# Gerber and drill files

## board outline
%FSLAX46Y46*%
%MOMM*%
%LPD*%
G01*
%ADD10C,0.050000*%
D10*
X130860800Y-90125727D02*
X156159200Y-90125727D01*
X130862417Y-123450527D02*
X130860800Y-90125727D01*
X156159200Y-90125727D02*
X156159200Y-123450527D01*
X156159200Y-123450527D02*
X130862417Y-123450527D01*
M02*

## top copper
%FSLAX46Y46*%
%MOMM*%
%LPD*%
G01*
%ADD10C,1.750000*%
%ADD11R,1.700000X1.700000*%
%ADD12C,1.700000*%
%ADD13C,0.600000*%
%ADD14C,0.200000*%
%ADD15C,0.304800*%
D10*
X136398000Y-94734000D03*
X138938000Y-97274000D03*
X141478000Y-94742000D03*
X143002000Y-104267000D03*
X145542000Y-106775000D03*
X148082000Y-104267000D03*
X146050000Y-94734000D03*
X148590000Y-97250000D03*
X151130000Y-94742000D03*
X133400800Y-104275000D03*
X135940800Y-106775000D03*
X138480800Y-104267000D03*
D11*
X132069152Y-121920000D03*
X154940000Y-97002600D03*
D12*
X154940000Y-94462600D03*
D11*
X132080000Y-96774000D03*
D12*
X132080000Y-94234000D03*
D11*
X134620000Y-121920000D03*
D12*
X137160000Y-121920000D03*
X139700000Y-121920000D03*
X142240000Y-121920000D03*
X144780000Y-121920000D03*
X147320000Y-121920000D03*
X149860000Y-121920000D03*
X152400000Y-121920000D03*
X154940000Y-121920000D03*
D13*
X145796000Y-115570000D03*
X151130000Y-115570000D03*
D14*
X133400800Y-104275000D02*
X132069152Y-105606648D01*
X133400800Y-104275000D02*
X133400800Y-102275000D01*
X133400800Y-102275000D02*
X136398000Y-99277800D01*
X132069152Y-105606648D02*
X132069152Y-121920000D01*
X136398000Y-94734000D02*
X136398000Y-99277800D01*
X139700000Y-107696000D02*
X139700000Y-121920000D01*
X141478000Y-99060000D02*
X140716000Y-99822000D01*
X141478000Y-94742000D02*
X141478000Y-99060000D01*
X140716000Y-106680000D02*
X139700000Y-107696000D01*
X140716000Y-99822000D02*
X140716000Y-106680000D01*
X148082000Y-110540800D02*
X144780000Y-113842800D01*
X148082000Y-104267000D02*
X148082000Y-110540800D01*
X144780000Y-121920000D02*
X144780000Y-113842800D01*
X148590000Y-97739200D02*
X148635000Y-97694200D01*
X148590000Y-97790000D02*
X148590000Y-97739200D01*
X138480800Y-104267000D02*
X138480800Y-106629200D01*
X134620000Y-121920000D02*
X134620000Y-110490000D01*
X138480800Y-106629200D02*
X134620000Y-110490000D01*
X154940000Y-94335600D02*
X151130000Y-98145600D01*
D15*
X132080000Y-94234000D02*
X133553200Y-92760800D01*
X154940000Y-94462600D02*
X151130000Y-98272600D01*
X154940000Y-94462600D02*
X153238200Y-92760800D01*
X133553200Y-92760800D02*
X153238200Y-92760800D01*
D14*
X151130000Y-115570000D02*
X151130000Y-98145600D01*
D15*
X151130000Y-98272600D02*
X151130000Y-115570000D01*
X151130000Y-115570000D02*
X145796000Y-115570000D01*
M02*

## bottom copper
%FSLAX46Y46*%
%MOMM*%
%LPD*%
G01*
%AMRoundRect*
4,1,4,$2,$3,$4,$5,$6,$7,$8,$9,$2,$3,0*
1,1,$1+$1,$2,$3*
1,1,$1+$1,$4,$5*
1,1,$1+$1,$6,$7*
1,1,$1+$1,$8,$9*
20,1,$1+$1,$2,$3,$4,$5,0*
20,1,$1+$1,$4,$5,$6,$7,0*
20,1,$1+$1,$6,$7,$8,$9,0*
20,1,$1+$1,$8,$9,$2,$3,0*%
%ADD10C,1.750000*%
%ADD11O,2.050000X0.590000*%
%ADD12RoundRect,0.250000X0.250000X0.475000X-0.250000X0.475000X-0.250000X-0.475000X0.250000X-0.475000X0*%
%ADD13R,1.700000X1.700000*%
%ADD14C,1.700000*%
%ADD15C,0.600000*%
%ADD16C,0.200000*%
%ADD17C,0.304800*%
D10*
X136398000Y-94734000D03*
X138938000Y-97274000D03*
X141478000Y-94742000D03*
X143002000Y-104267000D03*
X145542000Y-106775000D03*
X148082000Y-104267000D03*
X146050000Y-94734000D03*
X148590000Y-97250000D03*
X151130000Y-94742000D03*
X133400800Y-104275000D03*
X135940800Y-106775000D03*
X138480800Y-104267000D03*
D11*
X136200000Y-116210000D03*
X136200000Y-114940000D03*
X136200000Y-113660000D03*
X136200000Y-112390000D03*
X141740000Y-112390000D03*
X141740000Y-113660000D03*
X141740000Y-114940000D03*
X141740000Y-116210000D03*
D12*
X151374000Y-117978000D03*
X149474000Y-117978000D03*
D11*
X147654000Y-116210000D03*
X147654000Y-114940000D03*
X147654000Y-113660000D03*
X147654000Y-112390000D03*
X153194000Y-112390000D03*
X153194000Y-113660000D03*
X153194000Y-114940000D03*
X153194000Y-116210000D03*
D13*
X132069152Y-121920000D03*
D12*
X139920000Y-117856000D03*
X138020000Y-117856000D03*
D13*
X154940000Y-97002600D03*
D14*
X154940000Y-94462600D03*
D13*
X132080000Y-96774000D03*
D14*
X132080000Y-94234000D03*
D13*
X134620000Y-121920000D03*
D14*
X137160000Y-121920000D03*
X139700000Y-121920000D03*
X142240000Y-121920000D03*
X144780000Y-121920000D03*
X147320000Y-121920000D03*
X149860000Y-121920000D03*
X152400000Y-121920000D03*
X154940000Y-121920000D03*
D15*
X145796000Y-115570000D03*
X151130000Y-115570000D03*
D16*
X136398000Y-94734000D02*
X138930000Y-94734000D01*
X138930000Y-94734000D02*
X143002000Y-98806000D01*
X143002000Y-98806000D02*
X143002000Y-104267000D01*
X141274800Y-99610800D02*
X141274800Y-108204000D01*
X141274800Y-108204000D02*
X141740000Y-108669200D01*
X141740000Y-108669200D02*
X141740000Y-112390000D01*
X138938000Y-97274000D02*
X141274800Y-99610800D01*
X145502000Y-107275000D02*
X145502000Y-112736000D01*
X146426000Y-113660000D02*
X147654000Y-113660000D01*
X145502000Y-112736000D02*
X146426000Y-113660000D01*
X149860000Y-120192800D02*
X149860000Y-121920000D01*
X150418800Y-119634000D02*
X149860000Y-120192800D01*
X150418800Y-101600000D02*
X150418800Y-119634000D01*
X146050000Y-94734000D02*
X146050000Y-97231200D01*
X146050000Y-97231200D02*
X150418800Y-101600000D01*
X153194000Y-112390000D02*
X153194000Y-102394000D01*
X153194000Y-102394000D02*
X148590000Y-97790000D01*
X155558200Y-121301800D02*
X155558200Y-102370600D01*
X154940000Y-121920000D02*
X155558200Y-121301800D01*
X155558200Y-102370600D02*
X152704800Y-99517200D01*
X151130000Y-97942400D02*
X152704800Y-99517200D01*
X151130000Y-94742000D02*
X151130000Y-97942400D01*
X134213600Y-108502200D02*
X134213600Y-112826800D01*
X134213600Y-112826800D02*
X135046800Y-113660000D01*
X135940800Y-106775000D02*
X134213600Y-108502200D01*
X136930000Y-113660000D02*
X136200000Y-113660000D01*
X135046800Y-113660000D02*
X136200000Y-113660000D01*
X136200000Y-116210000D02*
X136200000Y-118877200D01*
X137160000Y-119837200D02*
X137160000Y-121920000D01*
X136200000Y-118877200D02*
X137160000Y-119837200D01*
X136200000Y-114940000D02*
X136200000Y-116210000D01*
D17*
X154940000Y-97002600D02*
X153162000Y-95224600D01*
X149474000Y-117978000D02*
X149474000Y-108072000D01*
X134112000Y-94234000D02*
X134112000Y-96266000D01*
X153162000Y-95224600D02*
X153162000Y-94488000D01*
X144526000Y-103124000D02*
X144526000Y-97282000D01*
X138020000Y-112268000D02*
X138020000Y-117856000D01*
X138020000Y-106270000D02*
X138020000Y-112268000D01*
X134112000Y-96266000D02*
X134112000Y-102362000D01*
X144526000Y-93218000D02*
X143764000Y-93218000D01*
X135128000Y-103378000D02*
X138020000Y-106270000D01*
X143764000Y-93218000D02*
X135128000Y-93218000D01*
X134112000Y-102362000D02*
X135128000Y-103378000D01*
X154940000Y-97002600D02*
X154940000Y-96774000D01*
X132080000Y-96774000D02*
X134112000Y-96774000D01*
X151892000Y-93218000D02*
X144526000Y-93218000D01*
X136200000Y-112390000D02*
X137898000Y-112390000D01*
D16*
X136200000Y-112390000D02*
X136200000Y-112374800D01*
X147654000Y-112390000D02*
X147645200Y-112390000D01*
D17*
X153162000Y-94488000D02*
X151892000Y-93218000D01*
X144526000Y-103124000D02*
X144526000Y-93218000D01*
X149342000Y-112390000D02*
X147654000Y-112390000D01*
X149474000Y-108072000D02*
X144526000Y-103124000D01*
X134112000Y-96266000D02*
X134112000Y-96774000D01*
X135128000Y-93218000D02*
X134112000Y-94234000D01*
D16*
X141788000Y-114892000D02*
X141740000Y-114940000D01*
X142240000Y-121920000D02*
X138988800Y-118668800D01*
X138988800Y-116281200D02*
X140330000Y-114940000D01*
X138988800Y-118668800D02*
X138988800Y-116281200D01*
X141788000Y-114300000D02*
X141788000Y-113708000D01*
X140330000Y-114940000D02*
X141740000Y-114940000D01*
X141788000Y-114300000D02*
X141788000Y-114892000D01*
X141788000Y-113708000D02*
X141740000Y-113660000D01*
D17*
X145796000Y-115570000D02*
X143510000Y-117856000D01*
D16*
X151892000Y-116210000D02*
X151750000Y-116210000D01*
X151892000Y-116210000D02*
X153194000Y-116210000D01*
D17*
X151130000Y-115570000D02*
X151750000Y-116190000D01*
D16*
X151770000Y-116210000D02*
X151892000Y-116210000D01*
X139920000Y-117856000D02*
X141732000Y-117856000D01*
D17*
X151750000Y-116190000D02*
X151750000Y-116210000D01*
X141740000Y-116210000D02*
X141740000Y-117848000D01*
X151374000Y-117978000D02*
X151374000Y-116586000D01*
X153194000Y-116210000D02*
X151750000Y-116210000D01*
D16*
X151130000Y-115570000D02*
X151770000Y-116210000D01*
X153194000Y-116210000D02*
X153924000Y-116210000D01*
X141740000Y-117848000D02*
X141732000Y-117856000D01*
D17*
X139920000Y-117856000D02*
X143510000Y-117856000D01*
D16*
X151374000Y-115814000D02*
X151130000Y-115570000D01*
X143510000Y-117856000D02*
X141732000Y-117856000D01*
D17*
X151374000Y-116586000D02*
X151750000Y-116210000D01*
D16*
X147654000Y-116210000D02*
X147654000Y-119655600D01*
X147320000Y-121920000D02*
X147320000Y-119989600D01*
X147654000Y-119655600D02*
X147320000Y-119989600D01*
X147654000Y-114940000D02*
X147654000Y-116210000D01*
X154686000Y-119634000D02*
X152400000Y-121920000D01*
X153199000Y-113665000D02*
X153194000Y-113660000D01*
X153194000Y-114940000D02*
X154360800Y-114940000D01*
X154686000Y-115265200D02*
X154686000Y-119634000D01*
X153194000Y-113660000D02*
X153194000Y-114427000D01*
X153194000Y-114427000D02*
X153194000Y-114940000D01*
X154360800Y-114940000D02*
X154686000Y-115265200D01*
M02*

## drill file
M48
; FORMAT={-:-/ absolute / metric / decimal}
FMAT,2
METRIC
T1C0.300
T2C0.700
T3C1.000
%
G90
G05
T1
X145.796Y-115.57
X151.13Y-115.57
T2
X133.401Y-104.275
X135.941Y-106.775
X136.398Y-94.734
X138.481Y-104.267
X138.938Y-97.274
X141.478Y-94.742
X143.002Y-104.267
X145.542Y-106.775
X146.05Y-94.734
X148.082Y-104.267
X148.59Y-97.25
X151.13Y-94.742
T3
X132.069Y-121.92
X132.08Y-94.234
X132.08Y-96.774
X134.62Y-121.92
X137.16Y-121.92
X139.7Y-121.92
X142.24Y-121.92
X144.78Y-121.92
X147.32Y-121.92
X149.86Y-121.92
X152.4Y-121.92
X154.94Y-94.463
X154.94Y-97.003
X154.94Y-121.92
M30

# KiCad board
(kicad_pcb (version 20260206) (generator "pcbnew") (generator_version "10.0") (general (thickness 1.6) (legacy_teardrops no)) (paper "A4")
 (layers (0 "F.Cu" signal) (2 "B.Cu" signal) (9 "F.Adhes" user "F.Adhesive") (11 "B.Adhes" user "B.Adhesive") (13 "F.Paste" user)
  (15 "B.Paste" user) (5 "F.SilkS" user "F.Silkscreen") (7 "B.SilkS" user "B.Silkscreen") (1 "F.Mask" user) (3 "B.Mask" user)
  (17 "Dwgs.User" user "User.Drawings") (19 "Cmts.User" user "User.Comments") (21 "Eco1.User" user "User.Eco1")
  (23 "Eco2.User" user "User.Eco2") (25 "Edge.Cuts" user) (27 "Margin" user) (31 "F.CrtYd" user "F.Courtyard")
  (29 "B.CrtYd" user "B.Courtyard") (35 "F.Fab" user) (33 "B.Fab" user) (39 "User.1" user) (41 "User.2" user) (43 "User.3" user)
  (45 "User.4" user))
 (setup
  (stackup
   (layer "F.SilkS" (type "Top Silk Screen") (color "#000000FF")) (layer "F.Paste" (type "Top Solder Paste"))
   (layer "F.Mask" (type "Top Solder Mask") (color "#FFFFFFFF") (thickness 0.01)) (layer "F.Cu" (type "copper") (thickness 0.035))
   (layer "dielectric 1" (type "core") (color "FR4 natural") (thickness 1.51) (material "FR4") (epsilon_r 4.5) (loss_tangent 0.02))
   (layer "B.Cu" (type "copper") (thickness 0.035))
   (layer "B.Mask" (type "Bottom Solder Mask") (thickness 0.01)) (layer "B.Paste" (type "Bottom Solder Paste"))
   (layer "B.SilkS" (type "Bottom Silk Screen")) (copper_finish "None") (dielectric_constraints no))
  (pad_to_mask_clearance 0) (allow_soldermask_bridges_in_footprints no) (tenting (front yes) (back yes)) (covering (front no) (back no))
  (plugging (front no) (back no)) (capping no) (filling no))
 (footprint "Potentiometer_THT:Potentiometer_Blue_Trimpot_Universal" (layer "F.Cu") (at 141.478 95.242 90)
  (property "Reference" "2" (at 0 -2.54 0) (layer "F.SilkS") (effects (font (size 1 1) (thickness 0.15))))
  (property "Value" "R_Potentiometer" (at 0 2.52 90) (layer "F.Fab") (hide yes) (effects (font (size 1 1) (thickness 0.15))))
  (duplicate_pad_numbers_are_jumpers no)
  (pad "1" thru_hole circle (at 0.508 -5.08 90) (size 1.75 1.75) (drill 0.7) (layers "*.Cu" "*.Mask") (remove_unused_layers no)
   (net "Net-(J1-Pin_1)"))
  (pad "2" thru_hole circle (at -2.032 -2.54 90) (size 1.75 1.75) (drill 0.7) (layers "*.Cu" "*.Mask") (remove_unused_layers no)
   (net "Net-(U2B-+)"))
  (pad "3" thru_hole circle (at 0.5 0 90) (size 1.75 1.75) (drill 0.7) (layers "*.Cu" "*.Mask") (remove_unused_layers no)
   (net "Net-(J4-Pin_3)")))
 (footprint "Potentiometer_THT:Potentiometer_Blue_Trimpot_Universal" (layer "F.Cu") (at 148.082 104.775 90)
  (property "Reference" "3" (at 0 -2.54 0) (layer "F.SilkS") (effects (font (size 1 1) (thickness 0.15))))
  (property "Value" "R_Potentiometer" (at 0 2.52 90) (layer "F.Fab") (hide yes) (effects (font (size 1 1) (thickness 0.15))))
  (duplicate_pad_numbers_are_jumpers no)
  (pad "1" thru_hole circle (at 0.508 -5.08 90) (size 1.75 1.75) (drill 0.7) (layers "*.Cu" "*.Mask") (remove_unused_layers no)
   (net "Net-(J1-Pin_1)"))
  (pad "2" thru_hole circle (at -2 -2.54 90) (size 1.75 1.75) (drill 0.7) (layers "*.Cu" "*.Mask") (remove_unused_layers no)
   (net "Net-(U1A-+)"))
  (pad "3" thru_hole circle (at 0.508 0 90) (size 1.75 1.75) (drill 0.7) (layers "*.Cu" "*.Mask") (remove_unused_layers no)
   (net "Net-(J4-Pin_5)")))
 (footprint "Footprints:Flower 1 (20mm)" (layer "F.Cu") (at 154.2796 110.744)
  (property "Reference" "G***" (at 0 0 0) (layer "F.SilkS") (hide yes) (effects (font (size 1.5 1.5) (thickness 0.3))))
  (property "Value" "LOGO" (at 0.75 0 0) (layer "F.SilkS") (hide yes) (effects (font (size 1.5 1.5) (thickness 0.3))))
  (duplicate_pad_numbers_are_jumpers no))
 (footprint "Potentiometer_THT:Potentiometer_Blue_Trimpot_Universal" (layer "F.Cu") (at 151.13 95.25 90)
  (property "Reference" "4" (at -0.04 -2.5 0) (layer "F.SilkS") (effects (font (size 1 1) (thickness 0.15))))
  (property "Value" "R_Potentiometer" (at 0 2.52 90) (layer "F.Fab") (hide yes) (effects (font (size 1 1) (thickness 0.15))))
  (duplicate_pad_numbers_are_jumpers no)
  (pad "1" thru_hole circle (at 0.516 -5.08 90) (size 1.75 1.75) (drill 0.7) (layers "*.Cu" "*.Mask") (remove_unused_layers no)
   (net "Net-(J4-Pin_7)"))
  (pad "2" thru_hole circle (at -2 -2.54 90) (size 1.75 1.75) (drill 0.7) (layers "*.Cu" "*.Mask") (remove_unused_layers no)
   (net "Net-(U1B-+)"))
  (pad "3" thru_hole circle (at 0.508 0 90) (size 1.75 1.75) (drill 0.7) (layers "*.Cu" "*.Mask") (remove_unused_layers no)
   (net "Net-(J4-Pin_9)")))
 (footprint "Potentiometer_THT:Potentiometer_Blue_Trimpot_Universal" (layer "F.Cu") (at 138.4808 104.775 90)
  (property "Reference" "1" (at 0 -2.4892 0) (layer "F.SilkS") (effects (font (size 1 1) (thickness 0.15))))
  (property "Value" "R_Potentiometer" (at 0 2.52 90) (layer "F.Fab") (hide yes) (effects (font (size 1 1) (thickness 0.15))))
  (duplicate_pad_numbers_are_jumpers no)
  (pad "1" thru_hole circle (at 0.5 -5.08 90) (size 1.75 1.75) (drill 0.7) (layers "*.Cu" "*.Mask") (remove_unused_layers no)
   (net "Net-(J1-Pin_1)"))
  (pad "2" thru_hole circle (at -2 -2.54 90) (size 1.75 1.75) (drill 0.7) (layers "*.Cu" "*.Mask") (remove_unused_layers no)
   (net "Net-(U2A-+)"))
  (pad "3" thru_hole circle (at 0.508 0 90) (size 1.75 1.75) (drill 0.7) (layers "*.Cu" "*.Mask") (remove_unused_layers no)
   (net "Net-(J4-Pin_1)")))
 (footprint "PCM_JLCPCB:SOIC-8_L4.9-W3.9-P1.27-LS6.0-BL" (layer "B.Cu") (at 138.97 114.3 90)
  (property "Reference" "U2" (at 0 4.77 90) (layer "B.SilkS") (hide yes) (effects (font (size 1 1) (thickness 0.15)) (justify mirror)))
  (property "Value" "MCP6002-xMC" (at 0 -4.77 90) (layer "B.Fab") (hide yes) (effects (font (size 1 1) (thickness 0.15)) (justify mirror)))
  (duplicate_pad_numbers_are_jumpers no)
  (pad "1" smd oval (at -1.91 -2.77 90) (size 0.59 2.05) (layers "B.Cu" "B.Mask" "B.Paste") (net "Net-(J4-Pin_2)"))
  (pad "2" smd oval (at -0.64 -2.77 90) (size 0.59 2.05) (layers "B.Cu" "B.Mask" "B.Paste") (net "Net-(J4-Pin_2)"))
  (pad "3" smd oval (at 0.64 -2.77 90) (size 0.59 2.05) (layers "B.Cu" "B.Mask" "B.Paste") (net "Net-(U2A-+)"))
  (pad "4" smd oval (at 1.91 -2.77 90) (size 0.59 2.05) (layers "B.Cu" "B.Mask" "B.Paste") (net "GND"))
  (pad "5" smd oval (at 1.91 2.77 90) (size 0.59 2.05) (layers "B.Cu" "B.Mask" "B.Paste") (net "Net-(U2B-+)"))
  (pad "6" smd oval (at 0.64 2.77 90) (size 0.59 2.05) (layers "B.Cu" "B.Mask" "B.Paste") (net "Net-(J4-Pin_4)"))
  (pad "7" smd oval (at -0.64 2.77 90) (size 0.59 2.05) (layers "B.Cu" "B.Mask" "B.Paste") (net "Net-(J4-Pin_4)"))
  (pad "8" smd oval (at -1.91 2.77 90) (size 0.59 2.05) (layers "B.Cu" "B.Mask" "B.Paste") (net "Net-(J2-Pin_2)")))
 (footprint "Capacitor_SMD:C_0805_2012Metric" (layer "B.Cu") (at 150.424 117.978 180)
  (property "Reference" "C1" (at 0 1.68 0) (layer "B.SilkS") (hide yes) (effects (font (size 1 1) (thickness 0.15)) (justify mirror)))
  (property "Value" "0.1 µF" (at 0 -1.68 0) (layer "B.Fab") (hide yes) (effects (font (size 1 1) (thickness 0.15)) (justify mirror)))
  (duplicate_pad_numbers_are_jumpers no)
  (pad "1" smd roundrect (at -0.95 0 180) (size 1 1.45) (layers "B.Cu" "B.Mask" "B.Paste") (roundrect_rratio 0.25) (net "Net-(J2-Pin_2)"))
  (pad "2" smd roundrect (at 0.95 0 180) (size 1 1.45) (layers "B.Cu" "B.Mask" "B.Paste") (roundrect_rratio 0.25) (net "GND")))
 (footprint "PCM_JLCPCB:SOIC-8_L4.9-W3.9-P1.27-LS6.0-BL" (layer "B.Cu") (at 150.424 114.3 90)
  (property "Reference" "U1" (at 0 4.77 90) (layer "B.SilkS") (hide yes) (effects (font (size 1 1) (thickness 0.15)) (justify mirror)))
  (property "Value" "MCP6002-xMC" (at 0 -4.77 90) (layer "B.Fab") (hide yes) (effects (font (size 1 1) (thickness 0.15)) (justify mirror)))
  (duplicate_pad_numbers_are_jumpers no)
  (pad "1" smd oval (at -1.91 -2.77 90) (size 0.59 2.05) (layers "B.Cu" "B.Mask" "B.Paste") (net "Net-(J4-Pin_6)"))
  (pad "2" smd oval (at -0.64 -2.77 90) (size 0.59 2.05) (layers "B.Cu" "B.Mask" "B.Paste") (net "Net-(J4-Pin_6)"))
  (pad "3" smd oval (at 0.64 -2.77 90) (size 0.59 2.05) (layers "B.Cu" "B.Mask" "B.Paste") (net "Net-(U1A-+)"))
  (pad "4" smd oval (at 1.91 -2.77 90) (size 0.59 2.05) (layers "B.Cu" "B.Mask" "B.Paste") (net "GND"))
  (pad "5" smd oval (at 1.91 2.77 90) (size 0.59 2.05) (layers "B.Cu" "B.Mask" "B.Paste") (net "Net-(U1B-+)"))
  (pad "6" smd oval (at 0.64 2.77 90) (size 0.59 2.05) (layers "B.Cu" "B.Mask" "B.Paste") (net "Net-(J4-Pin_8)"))
  (pad "7" smd oval (at -0.64 2.77 90) (size 0.59 2.05) (layers "B.Cu" "B.Mask" "B.Paste") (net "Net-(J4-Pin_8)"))
  (pad "8" smd oval (at -1.91 2.77 90) (size 0.59 2.05) (layers "B.Cu" "B.Mask" "B.Paste") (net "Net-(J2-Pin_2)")))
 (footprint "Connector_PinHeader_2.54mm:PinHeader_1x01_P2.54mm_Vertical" (layer "B.Cu") (at 132.069152 121.92 -90)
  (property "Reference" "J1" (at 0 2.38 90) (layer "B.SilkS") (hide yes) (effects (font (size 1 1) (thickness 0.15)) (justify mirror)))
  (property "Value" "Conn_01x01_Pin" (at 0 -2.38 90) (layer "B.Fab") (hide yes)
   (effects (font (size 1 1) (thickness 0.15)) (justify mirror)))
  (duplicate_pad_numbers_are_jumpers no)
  (pad "1" thru_hole rect (at 0 0 270) (size 1.7 1.7) (drill 1) (layers "*.Cu" "*.Mask") (remove_unused_layers no) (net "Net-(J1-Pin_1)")))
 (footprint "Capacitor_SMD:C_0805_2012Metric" (layer "B.Cu") (at 138.97 117.856 180)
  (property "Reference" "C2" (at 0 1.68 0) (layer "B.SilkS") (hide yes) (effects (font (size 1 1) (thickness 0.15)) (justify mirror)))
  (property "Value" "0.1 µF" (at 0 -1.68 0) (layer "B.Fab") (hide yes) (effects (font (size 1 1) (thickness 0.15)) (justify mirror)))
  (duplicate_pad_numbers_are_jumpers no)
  (pad "1" smd roundrect (at -0.95 0 180) (size 1 1.45) (layers "B.Cu" "B.Mask" "B.Paste") (roundrect_rratio 0.25) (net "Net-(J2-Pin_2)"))
  (pad "2" smd roundrect (at 0.95 0 180) (size 1 1.45) (layers "B.Cu" "B.Mask" "B.Paste") (roundrect_rratio 0.25) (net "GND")))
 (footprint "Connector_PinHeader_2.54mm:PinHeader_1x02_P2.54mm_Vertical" (layer "B.Cu") (at 154.94 97.0026)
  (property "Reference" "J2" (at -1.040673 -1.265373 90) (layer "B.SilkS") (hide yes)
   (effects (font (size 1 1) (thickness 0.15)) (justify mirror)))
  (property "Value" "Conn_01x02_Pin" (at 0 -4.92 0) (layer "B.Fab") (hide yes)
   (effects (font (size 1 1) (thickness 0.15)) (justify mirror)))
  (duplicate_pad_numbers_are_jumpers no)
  (pad "1" thru_hole rect (at 0 0) (size 1.7 1.7) (drill 1) (layers "*.Cu" "*.Mask") (remove_unused_layers no) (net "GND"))
  (pad "2" thru_hole circle (at 0 -2.54) (size 1.7 1.7) (drill 1) (layers "*.Cu" "*.Mask") (remove_unused_layers no) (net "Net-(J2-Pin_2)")))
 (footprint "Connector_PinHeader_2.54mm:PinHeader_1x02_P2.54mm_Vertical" (layer "B.Cu") (at 132.08 96.774)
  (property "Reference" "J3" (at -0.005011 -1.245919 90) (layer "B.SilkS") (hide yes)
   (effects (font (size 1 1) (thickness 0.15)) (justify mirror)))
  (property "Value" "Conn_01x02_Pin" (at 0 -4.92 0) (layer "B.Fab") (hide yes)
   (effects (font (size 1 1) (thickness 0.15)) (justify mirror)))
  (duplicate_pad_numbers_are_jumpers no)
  (pad "1" thru_hole rect (at 0 0) (size 1.7 1.7) (drill 1) (layers "*.Cu" "*.Mask") (remove_unused_layers no) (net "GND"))
  (pad "2" thru_hole circle (at 0 -2.54) (size 1.7 1.7) (drill 1) (layers "*.Cu" "*.Mask") (remove_unused_layers no) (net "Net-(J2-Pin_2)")))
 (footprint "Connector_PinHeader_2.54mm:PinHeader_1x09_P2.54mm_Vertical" (layer "B.Cu") (at 134.62 121.92 -90)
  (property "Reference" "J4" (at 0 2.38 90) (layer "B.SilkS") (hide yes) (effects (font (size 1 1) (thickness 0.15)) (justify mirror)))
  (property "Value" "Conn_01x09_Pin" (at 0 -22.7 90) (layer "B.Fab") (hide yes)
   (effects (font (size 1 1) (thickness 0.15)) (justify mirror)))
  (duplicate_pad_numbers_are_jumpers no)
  (pad "1" thru_hole rect (at 0 0 270) (size 1.7 1.7) (drill 1) (layers "*.Cu" "*.Mask") (remove_unused_layers no) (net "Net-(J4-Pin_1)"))
  (pad "2" thru_hole circle (at 0 -2.54 270) (size 1.7 1.7) (drill 1) (layers "*.Cu" "*.Mask") (remove_unused_layers no)
   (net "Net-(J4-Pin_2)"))
  (pad "3" thru_hole circle (at 0 -5.08 270) (size 1.7 1.7) (drill 1) (layers "*.Cu" "*.Mask") (remove_unused_layers no)
   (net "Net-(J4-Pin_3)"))
  (pad "4" thru_hole circle (at 0 -7.62 270) (size 1.7 1.7) (drill 1) (layers "*.Cu" "*.Mask") (remove_unused_layers no)
   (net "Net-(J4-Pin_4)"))
  (pad "5" thru_hole circle (at 0 -10.16 270) (size 1.7 1.7) (drill 1) (layers "*.Cu" "*.Mask") (remove_unused_layers no)
   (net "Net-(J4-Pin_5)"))
  (pad "6" thru_hole circle (at 0 -12.7 270) (size 1.7 1.7) (drill 1) (layers "*.Cu" "*.Mask") (remove_unused_layers no)
   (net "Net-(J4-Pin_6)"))
  (pad "7" thru_hole circle (at 0 -15.24 270) (size 1.7 1.7) (drill 1) (layers "*.Cu" "*.Mask") (remove_unused_layers no)
   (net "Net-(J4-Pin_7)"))
  (pad "8" thru_hole circle (at 0 -17.78 270) (size 1.7 1.7) (drill 1) (layers "*.Cu" "*.Mask") (remove_unused_layers no)
   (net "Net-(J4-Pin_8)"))
  (pad "9" thru_hole circle (at 0 -20.32 270) (size 1.7 1.7) (drill 1) (layers "*.Cu" "*.Mask") (remove_unused_layers no)
   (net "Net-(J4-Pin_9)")))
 (gr_line (start 130.8608 90.125727) (end 156.1592 90.125727) (stroke (width 0.05) (type default)) (layer "Edge.Cuts"))
 (gr_line (start 130.862417 123.450527) (end 130.8608 90.125727) (stroke (width 0.05) (type default)) (layer "Edge.Cuts"))
 (gr_line (start 156.1592 90.125727) (end 156.1592 123.450527) (stroke (width 0.05) (type solid)) (layer "Edge.Cuts"))
 (gr_line (start 156.1592 123.450527) (end 130.862417 123.450527) (stroke (width 0.05) (type default)) (layer "Edge.Cuts"))
 (segment (start 133.4008 104.275) (end 132.069152 105.606648) (width 0.2) (layer "F.Cu") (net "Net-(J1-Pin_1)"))
 (segment (start 133.4008 104.275) (end 133.4008 102.275) (width 0.2) (layer "F.Cu") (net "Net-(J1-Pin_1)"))
 (segment (start 133.4008 102.275) (end 136.398 99.2778) (width 0.2) (layer "F.Cu") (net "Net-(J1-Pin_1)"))
 (segment (start 132.069152 105.606648) (end 132.069152 121.92) (width 0.2) (layer "F.Cu") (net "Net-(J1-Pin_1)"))
 (segment (start 136.398 94.734) (end 136.398 99.2778) (width 0.2) (layer "F.Cu") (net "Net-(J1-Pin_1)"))
 (segment (start 136.398 94.734) (end 138.93 94.734) (width 0.2) (layer "B.Cu") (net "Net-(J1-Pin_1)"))
 (segment (start 138.93 94.734) (end 143.002 98.806) (width 0.2) (layer "B.Cu") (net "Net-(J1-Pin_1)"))
 (segment (start 143.002 98.806) (end 143.002 104.267) (width 0.2) (layer "B.Cu") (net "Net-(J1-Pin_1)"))
 (segment (start 141.2748 99.6108) (end 141.2748 108.204) (width 0.2) (layer "B.Cu") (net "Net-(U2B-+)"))
 (segment (start 141.2748 108.204) (end 141.74 108.6692) (width 0.2) (layer "B.Cu") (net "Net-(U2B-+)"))
 (segment (start 141.74 108.6692) (end 141.74 112.39) (width 0.2) (layer "B.Cu") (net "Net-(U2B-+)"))
 (segment (start 138.938 97.274) (end 141.2748 99.6108) (width 0.2) (layer "B.Cu") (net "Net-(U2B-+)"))
 (segment (start 139.7 107.696) (end 139.7 121.92) (width 0.2) (layer "F.Cu") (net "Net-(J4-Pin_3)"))
 (segment (start 141.478 99.06) (end 140.716 99.822) (width 0.2) (layer "F.Cu") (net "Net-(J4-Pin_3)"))
 (segment (start 141.478 94.742) (end 141.478 99.06) (width 0.2) (layer "F.Cu") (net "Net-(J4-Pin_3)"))
 (segment (start 140.716 106.68) (end 139.7 107.696) (width 0.2) (layer "F.Cu") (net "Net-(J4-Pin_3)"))
 (segment (start 140.716 99.822) (end 140.716 106.68) (width 0.2) (layer "F.Cu") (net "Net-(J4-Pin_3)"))
 (segment (start 145.502 107.275) (end 145.502 112.736) (width 0.2) (layer "B.Cu") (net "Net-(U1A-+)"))
 (segment (start 146.426 113.66) (end 147.654 113.66) (width 0.2) (layer "B.Cu") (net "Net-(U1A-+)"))
 (segment (start 145.502 112.736) (end 146.426 113.66) (width 0.2) (layer "B.Cu") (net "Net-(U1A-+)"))
 (segment (start 148.082 110.5408) (end 144.78 113.8428) (width 0.2) (layer "F.Cu") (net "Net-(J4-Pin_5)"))
 (segment (start 148.082 104.267) (end 148.082 110.5408) (width 0.2) (layer "F.Cu") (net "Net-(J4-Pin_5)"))
 (segment (start 144.78 121.92) (end 144.78 113.8428) (width 0.2) (layer "F.Cu") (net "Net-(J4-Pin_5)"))
 (segment (start 149.86 120.1928) (end 149.86 121.92) (width 0.2) (layer "B.Cu") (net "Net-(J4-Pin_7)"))
 (segment (start 150.4188 119.634) (end 149.86 120.1928) (width 0.2) (layer "B.Cu") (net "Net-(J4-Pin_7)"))
 (segment (start 150.4188 101.6) (end 150.4188 119.634) (width 0.2) (layer "B.Cu") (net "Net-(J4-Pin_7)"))
 (segment (start 146.05 94.734) (end 146.05 97.2312) (width 0.2) (layer "B.Cu") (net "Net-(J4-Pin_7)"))
 (segment (start 146.05 97.2312) (end 150.4188 101.6) (width 0.2) (layer "B.Cu") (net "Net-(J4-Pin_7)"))
 (segment (start 148.59 97.7392) (end 148.635 97.6942) (width 0.2) (layer "F.Cu") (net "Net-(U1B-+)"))
 (segment (start 148.59 97.79) (end 148.59 97.7392) (width 0.2) (layer "F.Cu") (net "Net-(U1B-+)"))
 (segment (start 153.194 112.39) (end 153.194 102.394) (width 0.2) (layer "B.Cu") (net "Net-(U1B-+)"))
 (segment (start 153.194 102.394) (end 148.59 97.79) (width 0.2) (layer "B.Cu") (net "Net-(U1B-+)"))
 (segment (start 155.5582 121.3018) (end 155.5582 102.3706) (width 0.2) (layer "B.Cu") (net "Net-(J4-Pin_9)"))
 (segment (start 154.94 121.92) (end 155.5582 121.3018) (width 0.2) (layer "B.Cu") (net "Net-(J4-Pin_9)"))
 (segment (start 155.5582 102.3706) (end 152.7048 99.5172) (width 0.2) (layer "B.Cu") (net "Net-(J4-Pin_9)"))
 (segment (start 151.13 97.9424) (end 152.7048 99.5172) (width 0.2) (layer "B.Cu") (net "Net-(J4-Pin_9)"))
 (segment (start 151.13 94.742) (end 151.13 97.9424) (width 0.2) (layer "B.Cu") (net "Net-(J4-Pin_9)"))
 (segment (start 134.2136 108.5022) (end 134.2136 112.8268) (width 0.2) (layer "B.Cu") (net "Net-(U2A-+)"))
 (segment (start 134.2136 112.8268) (end 135.0468 113.66) (width 0.2) (layer "B.Cu") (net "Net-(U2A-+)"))
 (segment (start 135.9408 106.775) (end 134.2136 108.5022) (width 0.2) (layer "B.Cu") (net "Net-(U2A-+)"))
 (segment (start 136.93 113.66) (end 136.2 113.66) (width 0.2) (layer "B.Cu") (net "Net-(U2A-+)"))
 (segment (start 135.0468 113.66) (end 136.2 113.66) (width 0.2) (layer "B.Cu") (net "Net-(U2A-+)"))
 (segment (start 138.4808 104.267) (end 138.4808 106.6292) (width 0.2) (layer "F.Cu") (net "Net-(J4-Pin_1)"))
 (segment (start 134.62 121.92) (end 134.62 110.49) (width 0.2) (layer "F.Cu") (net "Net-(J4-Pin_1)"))
 (segment (start 138.4808 106.6292) (end 134.62 110.49) (width 0.2) (layer "F.Cu") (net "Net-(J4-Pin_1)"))
 (segment (start 136.2 116.21) (end 136.2 118.8772) (width 0.2) (layer "B.Cu") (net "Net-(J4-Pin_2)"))
 (segment (start 137.16 119.8372) (end 137.16 121.92) (width 0.2) (layer "B.Cu") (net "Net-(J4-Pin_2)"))
 (segment (start 136.2 118.8772) (end 137.16 119.8372) (width 0.2) (layer "B.Cu") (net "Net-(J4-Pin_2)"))
 (segment (start 136.2 114.94) (end 136.2 116.21) (width 0.2) (layer "B.Cu") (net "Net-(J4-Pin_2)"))
 (segment (start 154.94 97.0026) (end 153.162 95.2246) (width 0.3048) (layer "B.Cu") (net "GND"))
 (segment (start 149.474 117.978) (end 149.474 108.072) (width 0.3048) (layer "B.Cu") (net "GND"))
 (segment (start 134.112 94.234) (end 134.112 96.266) (width 0.3048) (layer "B.Cu") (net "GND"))
 (segment (start 153.162 95.2246) (end 153.162 94.488) (width 0.3048) (layer "B.Cu") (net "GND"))
 (segment (start 144.526 103.124) (end 144.526 97.282) (width 0.3048) (layer "B.Cu") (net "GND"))
 (segment (start 138.02 112.268) (end 138.02 117.856) (width 0.3048) (layer "B.Cu") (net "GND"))
 (segment (start 138.02 106.27) (end 138.02 112.268) (width 0.3048) (layer "B.Cu") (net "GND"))
 (segment (start 134.112 96.266) (end 134.112 102.362) (width 0.3048) (layer "B.Cu") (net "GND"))
 (segment (start 144.526 93.218) (end 143.764 93.218) (width 0.3048) (layer "B.Cu") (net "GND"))
 (segment (start 135.128 103.378) (end 138.02 106.27) (width 0.3048) (layer "B.Cu") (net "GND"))
 (segment (start 143.764 93.218) (end 135.128 93.218) (width 0.3048) (layer "B.Cu") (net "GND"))
 (segment (start 134.112 102.362) (end 135.128 103.378) (width 0.3048) (layer "B.Cu") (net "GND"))
 (segment (start 154.94 97.0026) (end 154.94 96.774) (width 0.3048) (layer "B.Cu") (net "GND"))
 (segment (start 132.08 96.774) (end 134.112 96.774) (width 0.3048) (layer "B.Cu") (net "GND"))
 (segment (start 151.892 93.218) (end 144.526 93.218) (width 0.3048) (layer "B.Cu") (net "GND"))
 (segment (start 136.2 112.39) (end 137.898 112.39) (width 0.3048) (layer "B.Cu") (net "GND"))
 (segment (start 136.2 112.39) (end 136.2 112.3748) (width 0.2) (layer "B.Cu") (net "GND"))
 (segment (start 147.654 112.39) (end 147.6452 112.39) (width 0.2) (layer "B.Cu") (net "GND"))
 (segment (start 153.162 94.488) (end 151.892 93.218) (width 0.3048) (layer "B.Cu") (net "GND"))
 (segment (start 144.526 103.124) (end 144.526 93.218) (width 0.3048) (layer "B.Cu") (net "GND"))
 (segment (start 149.342 112.39) (end 147.654 112.39) (width 0.3048) (layer "B.Cu") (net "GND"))
 (segment (start 149.474 108.072) (end 144.526 103.124) (width 0.3048) (layer "B.Cu") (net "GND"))
 (segment (start 134.112 96.266) (end 134.112 96.774) (width 0.3048) (layer "B.Cu") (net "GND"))
 (segment (start 135.128 93.218) (end 134.112 94.234) (width 0.3048) (layer "B.Cu") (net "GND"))
 (segment (start 141.788 114.892) (end 141.74 114.94) (width 0.2) (layer "B.Cu") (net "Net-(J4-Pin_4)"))
 (segment (start 142.24 121.92) (end 138.9888 118.6688) (width 0.2) (layer "B.Cu") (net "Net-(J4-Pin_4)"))
 (segment (start 138.9888 116.2812) (end 140.33 114.94) (width 0.2) (layer "B.Cu") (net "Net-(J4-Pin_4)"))
 (segment (start 138.9888 118.6688) (end 138.9888 116.2812) (width 0.2) (layer "B.Cu") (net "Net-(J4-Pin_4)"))
 (segment (start 141.788 114.3) (end 141.788 113.708) (width 0.2) (layer "B.Cu") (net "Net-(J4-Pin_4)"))
 (segment (start 140.33 114.94) (end 141.74 114.94) (width 0.2) (layer "B.Cu") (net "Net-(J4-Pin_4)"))
 (segment (start 141.788 114.3) (end 141.788 114.892) (width 0.2) (layer "B.Cu") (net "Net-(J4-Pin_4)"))
 (segment (start 141.788 113.708) (end 141.74 113.66) (width 0.2) (layer "B.Cu") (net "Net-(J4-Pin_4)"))
 (segment (start 154.94 94.3356) (end 151.13 98.1456) (width 0.2) (layer "F.Cu") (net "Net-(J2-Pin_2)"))
 (segment (start 132.08 94.234) (end 133.5532 92.7608) (width 0.3048) (layer "F.Cu") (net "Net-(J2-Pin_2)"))
 (segment (start 154.94 94.4626) (end 151.13 98.2726) (width 0.3048) (layer "F.Cu") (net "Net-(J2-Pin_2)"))
 (segment (start 154.94 94.4626) (end 153.2382 92.7608) (width 0.3048) (layer "F.Cu") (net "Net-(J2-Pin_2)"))
 (segment (start 133.5532 92.7608) (end 153.2382 92.7608) (width 0.3048) (layer "F.Cu") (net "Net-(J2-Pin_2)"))
 (segment (start 151.13 115.57) (end 151.13 98.1456) (width 0.2) (layer "F.Cu") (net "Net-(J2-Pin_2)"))
 (segment (start 151.13 98.2726) (end 151.13 115.57) (width 0.3048) (layer "F.Cu") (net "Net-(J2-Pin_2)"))
 (segment (start 151.13 115.57) (end 145.796 115.57) (width 0.3048) (layer "F.Cu") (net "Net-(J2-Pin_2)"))
 (via (at 145.796 115.57) (size 0.6) (drill 0.3) (layers "F.Cu" "B.Cu") (capping no) (covering (front no) (back no))
  (plugging (front no) (back no)) (filling no) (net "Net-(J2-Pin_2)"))
 (via (at 151.13 115.57) (size 0.6) (drill 0.3) (layers "F.Cu" "B.Cu") (capping no) (covering (front no) (back no))
  (plugging (front no) (back no)) (filling no) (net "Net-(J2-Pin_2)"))
 (segment (start 145.796 115.57) (end 143.51 117.856) (width 0.3048) (layer "B.Cu") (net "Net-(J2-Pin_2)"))
 (segment (start 151.892 116.21) (end 151.75 116.21) (width 0.2) (layer "B.Cu") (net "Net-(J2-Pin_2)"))
 (segment (start 151.892 116.21) (end 153.194 116.21) (width 0.2) (layer "B.Cu") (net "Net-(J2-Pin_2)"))
 (segment (start 151.13 115.57) (end 151.75 116.19) (width 0.3048) (layer "B.Cu") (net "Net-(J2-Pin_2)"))
 (segment (start 151.77 116.21) (end 151.892 116.21) (width 0.2) (layer "B.Cu") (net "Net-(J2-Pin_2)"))
 (segment (start 139.92 117.856) (end 141.732 117.856) (width 0.2) (layer "B.Cu") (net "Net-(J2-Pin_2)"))
 (segment (start 151.75 116.19) (end 151.75 116.21) (width 0.3048) (layer "B.Cu") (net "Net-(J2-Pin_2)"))
 (segment (start 141.74 116.21) (end 141.74 117.848) (width 0.3048) (layer "B.Cu") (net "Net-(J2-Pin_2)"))
 (segment (start 151.374 117.978) (end 151.374 116.586) (width 0.3048) (layer "B.Cu") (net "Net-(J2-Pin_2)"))
 (segment (start 153.194 116.21) (end 151.75 116.21) (width 0.3048) (layer "B.Cu") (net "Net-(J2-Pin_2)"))
 (segment (start 151.13 115.57) (end 151.77 116.21) (width 0.2) (layer "B.Cu") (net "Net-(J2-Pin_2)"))
 (segment (start 153.194 116.21) (end 153.924 116.21) (width 0.2) (layer "B.Cu") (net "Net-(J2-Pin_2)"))
 (segment (start 141.74 117.848) (end 141.732 117.856) (width 0.2) (layer "B.Cu") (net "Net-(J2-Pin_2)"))
 (segment (start 139.92 117.856) (end 143.51 117.856) (width 0.3048) (layer "B.Cu") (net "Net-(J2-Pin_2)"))
 (segment (start 151.374 115.814) (end 151.13 115.57) (width 0.2) (layer "B.Cu") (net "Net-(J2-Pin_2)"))
 (segment (start 143.51 117.856) (end 141.732 117.856) (width 0.2) (layer "B.Cu") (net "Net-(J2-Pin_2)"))
 (segment (start 151.374 116.586) (end 151.75 116.21) (width 0.3048) (layer "B.Cu") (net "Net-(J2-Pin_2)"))
 (segment (start 147.654 116.21) (end 147.654 119.6556) (width 0.2) (layer "B.Cu") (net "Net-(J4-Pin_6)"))
 (segment (start 147.32 121.92) (end 147.32 119.9896) (width 0.2) (layer "B.Cu") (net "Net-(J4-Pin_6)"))
 (segment (start 147.654 119.6556) (end 147.32 119.9896) (width 0.2) (layer "B.Cu") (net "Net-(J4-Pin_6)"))
 (segment (start 147.654 114.94) (end 147.654 116.21) (width 0.2) (layer "B.Cu") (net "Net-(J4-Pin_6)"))
 (segment (start 154.686 119.634) (end 152.4 121.92) (width 0.2) (layer "B.Cu") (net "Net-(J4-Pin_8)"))
 (segment (start 153.199 113.665) (end 153.194 113.66) (width 0.2) (layer "B.Cu") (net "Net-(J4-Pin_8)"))
 (segment (start 153.194 114.94) (end 154.3608 114.94) (width 0.2) (layer "B.Cu") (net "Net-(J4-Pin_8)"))
 (segment (start 154.686 115.2652) (end 154.686 119.634) (width 0.2) (layer "B.Cu") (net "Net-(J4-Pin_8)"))
 (segment (start 153.194 113.66) (end 153.194 114.427) (width 0.2) (layer "B.Cu") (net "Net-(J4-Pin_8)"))
 (segment (start 153.194 114.427) (end 153.194 114.94) (width 0.2) (layer "B.Cu") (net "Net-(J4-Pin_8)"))
 (segment (start 154.3608 114.94) (end 154.686 115.2652) (width 0.2) (layer "B.Cu") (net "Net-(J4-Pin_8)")))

